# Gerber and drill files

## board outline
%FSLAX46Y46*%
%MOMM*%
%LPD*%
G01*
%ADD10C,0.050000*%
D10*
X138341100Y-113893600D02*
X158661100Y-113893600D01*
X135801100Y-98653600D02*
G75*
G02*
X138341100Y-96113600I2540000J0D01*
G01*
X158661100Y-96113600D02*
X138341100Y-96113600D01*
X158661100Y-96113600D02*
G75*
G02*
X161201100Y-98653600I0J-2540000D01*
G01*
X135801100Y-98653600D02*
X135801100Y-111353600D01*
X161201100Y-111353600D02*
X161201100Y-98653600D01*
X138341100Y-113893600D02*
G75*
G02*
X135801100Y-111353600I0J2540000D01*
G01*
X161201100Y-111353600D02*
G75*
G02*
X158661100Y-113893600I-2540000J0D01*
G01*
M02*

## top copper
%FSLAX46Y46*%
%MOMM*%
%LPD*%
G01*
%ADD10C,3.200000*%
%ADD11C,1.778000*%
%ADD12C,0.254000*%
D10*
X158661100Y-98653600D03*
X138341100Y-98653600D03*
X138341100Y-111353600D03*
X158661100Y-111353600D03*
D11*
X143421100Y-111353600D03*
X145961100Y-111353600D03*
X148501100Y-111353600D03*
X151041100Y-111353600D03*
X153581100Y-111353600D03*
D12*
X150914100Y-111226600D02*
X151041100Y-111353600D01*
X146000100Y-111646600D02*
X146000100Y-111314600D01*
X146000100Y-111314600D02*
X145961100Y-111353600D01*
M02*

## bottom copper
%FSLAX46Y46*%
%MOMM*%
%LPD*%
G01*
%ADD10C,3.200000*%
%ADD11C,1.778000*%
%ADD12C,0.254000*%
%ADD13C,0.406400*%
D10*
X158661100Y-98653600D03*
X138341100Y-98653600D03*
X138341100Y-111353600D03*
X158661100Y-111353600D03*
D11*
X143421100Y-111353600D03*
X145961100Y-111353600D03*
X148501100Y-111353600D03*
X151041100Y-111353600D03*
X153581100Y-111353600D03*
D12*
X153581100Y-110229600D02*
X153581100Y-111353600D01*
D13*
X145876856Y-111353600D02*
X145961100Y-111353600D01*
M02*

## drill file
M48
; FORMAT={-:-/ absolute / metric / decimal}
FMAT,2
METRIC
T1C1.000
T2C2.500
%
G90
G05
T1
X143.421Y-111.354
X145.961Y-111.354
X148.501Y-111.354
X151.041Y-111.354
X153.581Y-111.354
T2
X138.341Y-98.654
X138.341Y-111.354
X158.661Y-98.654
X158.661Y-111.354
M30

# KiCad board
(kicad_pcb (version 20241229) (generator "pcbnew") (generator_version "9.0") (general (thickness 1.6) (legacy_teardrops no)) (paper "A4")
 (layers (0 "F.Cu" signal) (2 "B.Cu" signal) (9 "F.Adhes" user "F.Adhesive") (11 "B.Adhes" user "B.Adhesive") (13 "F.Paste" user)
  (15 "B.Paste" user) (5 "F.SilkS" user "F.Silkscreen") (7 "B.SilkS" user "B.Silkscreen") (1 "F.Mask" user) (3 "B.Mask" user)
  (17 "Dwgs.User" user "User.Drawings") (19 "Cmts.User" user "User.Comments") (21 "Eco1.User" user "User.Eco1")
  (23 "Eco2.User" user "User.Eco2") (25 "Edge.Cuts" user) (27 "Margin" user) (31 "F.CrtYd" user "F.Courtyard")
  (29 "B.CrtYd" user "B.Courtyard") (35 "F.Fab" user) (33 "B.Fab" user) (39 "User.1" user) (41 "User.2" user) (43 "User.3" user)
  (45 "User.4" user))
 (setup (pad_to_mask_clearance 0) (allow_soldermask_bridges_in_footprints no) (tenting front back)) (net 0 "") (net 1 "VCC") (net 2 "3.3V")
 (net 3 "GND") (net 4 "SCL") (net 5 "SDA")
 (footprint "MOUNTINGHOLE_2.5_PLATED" (layer "F.Cu") (at 158.6611 98.6536)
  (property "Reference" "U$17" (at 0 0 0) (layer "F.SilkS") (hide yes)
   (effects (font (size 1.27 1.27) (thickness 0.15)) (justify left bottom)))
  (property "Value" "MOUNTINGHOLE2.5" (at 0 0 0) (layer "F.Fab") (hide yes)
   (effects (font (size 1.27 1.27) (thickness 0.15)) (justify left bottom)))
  (pad "P$1" thru_hole circle (at 0 0) (size 3.2 3.2) (drill 2.5) (layers "*.Cu" "*.Mask") (remove_unused_layers no)
   (solder_mask_margin 0.0508) (thermal_bridge_angle 0))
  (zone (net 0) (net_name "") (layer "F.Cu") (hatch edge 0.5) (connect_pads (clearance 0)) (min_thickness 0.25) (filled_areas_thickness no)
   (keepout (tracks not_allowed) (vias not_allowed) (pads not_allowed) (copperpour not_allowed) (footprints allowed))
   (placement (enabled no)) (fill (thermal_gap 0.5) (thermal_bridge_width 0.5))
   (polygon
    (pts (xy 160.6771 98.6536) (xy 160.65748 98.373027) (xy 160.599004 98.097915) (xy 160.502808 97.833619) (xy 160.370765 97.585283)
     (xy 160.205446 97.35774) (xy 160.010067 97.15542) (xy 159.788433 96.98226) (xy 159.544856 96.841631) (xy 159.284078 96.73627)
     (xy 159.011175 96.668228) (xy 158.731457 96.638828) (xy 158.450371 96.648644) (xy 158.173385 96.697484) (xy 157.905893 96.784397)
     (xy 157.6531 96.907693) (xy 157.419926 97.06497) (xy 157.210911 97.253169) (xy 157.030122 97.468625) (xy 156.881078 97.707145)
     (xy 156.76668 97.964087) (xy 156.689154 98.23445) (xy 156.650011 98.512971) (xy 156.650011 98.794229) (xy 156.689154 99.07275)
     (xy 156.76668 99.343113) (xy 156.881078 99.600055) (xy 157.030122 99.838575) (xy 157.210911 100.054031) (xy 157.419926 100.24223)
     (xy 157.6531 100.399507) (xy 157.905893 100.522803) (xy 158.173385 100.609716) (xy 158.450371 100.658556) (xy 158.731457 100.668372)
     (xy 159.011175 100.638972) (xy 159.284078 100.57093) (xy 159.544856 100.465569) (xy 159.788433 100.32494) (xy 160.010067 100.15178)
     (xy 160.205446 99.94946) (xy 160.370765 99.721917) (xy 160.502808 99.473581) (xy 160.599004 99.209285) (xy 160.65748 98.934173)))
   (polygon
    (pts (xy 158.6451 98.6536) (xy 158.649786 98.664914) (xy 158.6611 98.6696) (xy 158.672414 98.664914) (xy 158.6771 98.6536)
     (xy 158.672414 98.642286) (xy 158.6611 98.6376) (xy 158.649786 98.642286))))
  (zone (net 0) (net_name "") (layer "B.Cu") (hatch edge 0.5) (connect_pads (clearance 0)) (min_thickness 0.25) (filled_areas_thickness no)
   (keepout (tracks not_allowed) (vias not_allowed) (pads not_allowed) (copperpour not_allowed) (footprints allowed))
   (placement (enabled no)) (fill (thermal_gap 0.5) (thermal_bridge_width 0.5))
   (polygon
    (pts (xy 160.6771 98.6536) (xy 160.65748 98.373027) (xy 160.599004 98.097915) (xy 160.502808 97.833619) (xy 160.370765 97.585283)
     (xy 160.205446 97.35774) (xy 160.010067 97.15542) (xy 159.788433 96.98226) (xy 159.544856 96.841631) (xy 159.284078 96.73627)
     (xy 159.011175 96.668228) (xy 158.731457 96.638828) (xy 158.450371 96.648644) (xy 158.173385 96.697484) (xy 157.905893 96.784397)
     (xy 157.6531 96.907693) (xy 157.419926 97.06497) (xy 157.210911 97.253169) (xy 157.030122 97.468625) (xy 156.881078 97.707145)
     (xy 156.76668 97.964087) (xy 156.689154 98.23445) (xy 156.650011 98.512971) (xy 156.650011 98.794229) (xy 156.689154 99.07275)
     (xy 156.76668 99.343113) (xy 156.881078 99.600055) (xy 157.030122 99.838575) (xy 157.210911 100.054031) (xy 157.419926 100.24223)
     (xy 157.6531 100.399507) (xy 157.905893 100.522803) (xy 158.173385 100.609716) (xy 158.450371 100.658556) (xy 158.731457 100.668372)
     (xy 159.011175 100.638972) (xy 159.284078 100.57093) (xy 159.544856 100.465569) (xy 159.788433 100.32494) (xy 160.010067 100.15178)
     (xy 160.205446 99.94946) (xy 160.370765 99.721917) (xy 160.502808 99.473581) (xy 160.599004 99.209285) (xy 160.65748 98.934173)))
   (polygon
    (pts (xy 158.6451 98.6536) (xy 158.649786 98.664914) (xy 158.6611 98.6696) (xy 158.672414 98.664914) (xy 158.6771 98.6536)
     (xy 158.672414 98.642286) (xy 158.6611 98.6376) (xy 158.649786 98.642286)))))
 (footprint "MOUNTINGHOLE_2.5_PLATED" (layer "F.Cu") (at 138.3411 98.6536)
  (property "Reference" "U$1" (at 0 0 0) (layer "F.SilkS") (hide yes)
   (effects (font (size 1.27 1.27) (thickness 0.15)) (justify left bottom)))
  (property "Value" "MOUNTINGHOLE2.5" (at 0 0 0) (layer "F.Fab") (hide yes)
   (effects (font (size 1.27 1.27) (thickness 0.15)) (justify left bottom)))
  (pad "P$1" thru_hole circle (at 0 0) (size 3.2 3.2) (drill 2.5) (layers "*.Cu" "*.Mask") (remove_unused_layers no)
   (solder_mask_margin 0.0508) (thermal_bridge_angle 0))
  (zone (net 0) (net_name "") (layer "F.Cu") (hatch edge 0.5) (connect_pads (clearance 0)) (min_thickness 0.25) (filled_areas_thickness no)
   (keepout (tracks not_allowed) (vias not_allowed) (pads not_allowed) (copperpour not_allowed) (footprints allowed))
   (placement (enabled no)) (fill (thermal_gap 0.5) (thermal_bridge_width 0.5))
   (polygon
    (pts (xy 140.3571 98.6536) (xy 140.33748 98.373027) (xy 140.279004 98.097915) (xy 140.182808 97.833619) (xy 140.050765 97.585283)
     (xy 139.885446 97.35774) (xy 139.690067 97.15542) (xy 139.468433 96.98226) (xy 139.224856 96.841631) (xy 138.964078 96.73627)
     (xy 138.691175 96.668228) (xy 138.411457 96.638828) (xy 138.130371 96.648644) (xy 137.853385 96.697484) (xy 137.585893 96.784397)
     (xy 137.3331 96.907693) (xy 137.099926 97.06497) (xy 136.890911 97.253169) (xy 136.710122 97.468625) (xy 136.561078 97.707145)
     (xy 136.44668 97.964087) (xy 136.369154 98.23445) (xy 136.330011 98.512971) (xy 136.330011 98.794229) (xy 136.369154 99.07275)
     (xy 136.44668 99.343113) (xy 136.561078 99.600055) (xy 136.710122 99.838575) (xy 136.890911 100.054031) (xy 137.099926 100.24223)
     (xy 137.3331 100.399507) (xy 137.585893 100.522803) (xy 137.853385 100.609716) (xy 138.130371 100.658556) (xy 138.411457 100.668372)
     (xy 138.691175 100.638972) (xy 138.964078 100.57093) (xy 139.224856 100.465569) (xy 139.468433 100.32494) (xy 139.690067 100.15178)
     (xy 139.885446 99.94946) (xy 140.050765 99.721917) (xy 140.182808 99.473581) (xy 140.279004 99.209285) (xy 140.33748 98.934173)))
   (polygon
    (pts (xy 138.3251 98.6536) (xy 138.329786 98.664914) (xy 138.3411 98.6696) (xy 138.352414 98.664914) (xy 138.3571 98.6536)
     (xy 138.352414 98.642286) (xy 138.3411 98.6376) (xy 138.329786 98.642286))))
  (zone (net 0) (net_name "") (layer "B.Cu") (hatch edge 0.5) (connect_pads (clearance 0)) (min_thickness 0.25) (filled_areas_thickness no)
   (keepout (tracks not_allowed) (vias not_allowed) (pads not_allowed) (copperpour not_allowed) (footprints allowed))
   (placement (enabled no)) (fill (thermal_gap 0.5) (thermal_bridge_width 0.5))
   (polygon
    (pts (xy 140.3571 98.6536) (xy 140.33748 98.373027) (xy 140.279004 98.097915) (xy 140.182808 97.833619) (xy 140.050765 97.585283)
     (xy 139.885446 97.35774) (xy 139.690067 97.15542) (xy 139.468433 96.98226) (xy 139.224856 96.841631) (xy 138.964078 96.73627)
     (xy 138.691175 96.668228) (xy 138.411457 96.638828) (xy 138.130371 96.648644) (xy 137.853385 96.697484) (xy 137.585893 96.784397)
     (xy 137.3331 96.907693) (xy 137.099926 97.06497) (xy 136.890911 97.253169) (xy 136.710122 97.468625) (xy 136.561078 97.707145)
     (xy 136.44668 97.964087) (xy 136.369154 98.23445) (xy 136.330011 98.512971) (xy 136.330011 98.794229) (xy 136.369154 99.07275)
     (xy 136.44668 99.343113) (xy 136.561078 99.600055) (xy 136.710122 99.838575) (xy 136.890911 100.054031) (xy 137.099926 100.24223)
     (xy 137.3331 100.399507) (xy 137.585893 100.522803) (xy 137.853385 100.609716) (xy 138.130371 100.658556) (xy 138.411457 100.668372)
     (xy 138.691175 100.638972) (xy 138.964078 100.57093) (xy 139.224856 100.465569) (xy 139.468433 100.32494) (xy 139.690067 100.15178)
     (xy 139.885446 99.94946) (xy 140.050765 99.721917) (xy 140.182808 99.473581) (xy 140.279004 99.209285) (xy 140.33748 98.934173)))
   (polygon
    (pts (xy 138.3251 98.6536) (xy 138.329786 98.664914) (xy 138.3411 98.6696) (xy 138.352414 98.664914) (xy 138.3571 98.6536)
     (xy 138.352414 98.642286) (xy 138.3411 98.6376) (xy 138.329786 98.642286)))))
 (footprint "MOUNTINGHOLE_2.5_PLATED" (layer "F.Cu") (at 138.3411 111.3536)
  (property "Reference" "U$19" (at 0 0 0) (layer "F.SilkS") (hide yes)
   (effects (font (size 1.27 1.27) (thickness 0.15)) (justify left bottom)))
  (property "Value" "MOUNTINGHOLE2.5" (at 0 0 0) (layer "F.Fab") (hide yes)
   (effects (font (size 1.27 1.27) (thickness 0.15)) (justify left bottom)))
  (pad "P$1" thru_hole circle (at 0 0) (size 3.2 3.2) (drill 2.5) (layers "*.Cu" "*.Mask") (remove_unused_layers no)
   (solder_mask_margin 0.0508) (thermal_bridge_angle 0))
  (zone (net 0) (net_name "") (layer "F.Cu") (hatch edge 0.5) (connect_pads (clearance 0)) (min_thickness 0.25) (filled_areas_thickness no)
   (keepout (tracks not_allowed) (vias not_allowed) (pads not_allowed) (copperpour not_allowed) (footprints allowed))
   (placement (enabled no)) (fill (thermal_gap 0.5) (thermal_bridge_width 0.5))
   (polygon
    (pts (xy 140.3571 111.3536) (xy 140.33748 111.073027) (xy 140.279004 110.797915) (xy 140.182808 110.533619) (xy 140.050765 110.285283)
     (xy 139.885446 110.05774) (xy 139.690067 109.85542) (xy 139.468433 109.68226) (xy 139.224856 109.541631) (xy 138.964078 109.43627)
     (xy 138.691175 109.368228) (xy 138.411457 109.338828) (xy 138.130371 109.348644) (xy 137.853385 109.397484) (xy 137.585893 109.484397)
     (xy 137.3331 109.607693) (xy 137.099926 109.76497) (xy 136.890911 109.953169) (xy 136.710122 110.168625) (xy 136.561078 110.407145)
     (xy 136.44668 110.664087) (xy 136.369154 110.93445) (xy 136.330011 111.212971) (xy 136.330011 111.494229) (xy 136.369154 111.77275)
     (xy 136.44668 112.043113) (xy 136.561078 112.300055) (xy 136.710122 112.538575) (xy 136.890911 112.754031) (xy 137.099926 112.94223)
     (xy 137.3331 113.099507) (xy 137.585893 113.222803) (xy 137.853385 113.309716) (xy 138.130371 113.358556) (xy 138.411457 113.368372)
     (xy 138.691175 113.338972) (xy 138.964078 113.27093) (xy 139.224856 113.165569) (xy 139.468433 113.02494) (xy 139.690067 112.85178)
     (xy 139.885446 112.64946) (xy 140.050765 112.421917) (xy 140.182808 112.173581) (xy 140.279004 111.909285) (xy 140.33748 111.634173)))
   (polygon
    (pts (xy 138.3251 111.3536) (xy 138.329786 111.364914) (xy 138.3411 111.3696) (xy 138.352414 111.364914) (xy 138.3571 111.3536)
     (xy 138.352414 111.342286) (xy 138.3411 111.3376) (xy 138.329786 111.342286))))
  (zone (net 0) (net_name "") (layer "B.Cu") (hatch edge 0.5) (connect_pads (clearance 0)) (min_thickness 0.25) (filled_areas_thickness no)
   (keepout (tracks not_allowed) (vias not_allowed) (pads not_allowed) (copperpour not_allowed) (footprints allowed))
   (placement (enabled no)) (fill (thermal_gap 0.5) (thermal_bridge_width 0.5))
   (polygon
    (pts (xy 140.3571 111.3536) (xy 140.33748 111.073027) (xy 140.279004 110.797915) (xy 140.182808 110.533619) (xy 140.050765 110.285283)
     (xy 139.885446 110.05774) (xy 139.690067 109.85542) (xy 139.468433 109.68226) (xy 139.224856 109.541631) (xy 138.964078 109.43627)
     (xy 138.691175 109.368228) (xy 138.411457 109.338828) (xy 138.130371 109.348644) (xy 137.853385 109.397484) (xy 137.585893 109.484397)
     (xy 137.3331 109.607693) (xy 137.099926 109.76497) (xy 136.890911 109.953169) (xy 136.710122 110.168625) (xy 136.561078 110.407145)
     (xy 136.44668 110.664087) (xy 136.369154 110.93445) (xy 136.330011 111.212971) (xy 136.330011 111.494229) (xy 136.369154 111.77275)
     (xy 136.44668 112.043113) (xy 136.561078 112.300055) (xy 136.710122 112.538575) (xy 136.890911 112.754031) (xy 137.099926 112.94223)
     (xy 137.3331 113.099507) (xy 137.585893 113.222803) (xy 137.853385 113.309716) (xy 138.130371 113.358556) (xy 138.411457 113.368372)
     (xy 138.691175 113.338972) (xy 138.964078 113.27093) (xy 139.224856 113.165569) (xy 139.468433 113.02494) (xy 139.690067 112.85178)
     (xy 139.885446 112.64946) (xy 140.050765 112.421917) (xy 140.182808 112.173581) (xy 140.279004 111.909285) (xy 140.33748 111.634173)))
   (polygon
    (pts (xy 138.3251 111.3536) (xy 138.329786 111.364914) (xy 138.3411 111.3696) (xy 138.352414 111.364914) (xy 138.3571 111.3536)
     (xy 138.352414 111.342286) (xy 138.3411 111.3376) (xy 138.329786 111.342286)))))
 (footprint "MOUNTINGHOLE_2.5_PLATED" (layer "F.Cu") (at 158.6611 111.3536)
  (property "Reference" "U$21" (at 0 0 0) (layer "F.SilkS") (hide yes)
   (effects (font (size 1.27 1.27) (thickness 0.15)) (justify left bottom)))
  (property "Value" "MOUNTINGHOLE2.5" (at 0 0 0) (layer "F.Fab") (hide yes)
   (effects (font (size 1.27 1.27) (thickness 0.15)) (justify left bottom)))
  (pad "P$1" thru_hole circle (at 0 0) (size 3.2 3.2) (drill 2.5) (layers "*.Cu" "*.Mask") (remove_unused_layers no)
   (solder_mask_margin 0.0508) (thermal_bridge_angle 0))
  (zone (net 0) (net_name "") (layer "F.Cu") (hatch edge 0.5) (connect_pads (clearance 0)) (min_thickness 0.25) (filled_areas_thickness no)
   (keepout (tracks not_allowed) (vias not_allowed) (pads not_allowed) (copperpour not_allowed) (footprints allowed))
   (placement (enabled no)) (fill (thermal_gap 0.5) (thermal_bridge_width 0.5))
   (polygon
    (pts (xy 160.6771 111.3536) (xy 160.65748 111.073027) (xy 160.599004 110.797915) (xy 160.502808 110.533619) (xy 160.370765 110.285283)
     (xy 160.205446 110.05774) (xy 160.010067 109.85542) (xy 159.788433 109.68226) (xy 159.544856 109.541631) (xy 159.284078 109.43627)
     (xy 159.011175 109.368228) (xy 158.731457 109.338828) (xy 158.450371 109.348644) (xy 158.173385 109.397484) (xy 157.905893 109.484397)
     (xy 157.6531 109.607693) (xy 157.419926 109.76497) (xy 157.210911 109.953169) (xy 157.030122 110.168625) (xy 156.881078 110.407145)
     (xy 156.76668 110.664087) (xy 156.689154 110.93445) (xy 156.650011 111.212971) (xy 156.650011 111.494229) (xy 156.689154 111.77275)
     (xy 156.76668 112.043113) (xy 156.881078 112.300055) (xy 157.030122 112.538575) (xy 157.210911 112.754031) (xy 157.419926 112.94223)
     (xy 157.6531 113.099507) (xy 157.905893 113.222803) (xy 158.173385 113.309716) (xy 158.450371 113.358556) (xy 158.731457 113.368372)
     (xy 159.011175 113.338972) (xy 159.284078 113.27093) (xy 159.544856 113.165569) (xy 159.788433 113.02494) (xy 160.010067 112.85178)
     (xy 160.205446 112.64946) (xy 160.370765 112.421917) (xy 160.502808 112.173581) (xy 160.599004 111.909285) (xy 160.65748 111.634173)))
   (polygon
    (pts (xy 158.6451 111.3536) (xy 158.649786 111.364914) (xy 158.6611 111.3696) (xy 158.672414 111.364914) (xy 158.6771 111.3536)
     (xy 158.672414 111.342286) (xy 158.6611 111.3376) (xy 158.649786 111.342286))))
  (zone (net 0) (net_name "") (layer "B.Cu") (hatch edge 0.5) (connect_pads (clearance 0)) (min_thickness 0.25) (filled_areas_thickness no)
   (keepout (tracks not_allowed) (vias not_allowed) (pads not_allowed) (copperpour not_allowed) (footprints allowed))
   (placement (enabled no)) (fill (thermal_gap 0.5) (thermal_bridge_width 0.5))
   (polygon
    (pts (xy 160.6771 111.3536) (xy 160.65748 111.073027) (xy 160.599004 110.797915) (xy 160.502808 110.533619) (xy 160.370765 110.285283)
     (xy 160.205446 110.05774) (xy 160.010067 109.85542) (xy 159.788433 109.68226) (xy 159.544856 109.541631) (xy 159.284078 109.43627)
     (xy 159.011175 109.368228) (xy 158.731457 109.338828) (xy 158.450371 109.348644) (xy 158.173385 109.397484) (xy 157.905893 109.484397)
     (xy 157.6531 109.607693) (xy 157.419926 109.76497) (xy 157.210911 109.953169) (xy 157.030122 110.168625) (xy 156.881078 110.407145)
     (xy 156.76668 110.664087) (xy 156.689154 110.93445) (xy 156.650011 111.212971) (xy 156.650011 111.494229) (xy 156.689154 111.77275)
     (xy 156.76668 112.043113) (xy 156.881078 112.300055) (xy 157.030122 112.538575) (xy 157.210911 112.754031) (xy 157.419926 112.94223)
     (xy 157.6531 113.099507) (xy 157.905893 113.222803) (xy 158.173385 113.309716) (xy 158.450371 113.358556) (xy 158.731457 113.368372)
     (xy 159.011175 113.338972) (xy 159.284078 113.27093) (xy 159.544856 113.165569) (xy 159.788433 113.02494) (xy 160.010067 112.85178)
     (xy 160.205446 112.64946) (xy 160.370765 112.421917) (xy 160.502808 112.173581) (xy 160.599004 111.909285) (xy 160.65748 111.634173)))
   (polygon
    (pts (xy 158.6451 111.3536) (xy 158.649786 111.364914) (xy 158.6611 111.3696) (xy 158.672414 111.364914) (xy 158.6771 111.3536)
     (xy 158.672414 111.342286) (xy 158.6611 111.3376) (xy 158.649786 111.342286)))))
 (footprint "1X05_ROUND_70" (layer "F.Cu") (at 148.5011 111.3536)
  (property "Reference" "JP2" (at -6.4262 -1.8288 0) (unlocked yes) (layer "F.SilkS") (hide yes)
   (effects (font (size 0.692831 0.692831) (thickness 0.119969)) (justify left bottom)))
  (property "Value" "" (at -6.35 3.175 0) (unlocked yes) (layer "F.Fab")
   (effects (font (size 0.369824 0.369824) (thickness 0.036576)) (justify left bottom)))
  (pad "1" thru_hole circle (at -5.08 0 90) (size 1.778 1.778) (drill 1) (layers "*.Cu" "*.Mask") (remove_unused_layers no) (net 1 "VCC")
   (solder_mask_margin 0.0508) (thermal_bridge_angle 0))
  (pad "2" thru_hole circle (at -2.54 0 90) (size 1.778 1.778) (drill 1) (layers "*.Cu" "*.Mask") (remove_unused_layers no) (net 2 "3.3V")
   (solder_mask_margin 0.0508) (thermal_bridge_angle 0))
  (pad "3" thru_hole circle (at 0 0 90) (size 1.778 1.778) (drill 1) (layers "*.Cu" "*.Mask") (remove_unused_layers no) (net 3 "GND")
   (solder_mask_margin 0.0508) (thermal_bridge_angle 0))
  (pad "4" thru_hole circle (at 2.54 0 90) (size 1.778 1.778) (drill 1) (layers "*.Cu" "*.Mask") (remove_unused_layers no) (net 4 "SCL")
   (solder_mask_margin 0.0508) (thermal_bridge_angle 0))
  (pad "5" thru_hole circle (at 5.08 0 90) (size 1.778 1.778) (drill 1) (layers "*.Cu" "*.Mask") (remove_unused_layers no) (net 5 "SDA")
   (solder_mask_margin 0.0508) (thermal_bridge_angle 0)))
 (gr_line (start 138.3411 113.8936) (end 158.6611 113.8936) (stroke (width 0.05) (type solid)) (layer "Edge.Cuts"))
 (gr_arc (start 135.8011 98.6536) (mid 136.545049 96.857549) (end 138.3411 96.1136) (stroke (width 0.05) (type solid)) (layer "Edge.Cuts"))
 (gr_line (start 158.6611 96.1136) (end 138.3411 96.1136) (stroke (width 0.05) (type solid)) (layer "Edge.Cuts"))
 (gr_arc (start 158.6611 96.1136) (mid 160.457151 96.857549) (end 161.2011 98.6536) (stroke (width 0.05) (type solid)) (layer "Edge.Cuts"))
 (gr_line (start 135.8011 98.6536) (end 135.8011 111.3536) (stroke (width 0.05) (type solid)) (layer "Edge.Cuts"))
 (gr_line (start 161.2011 111.3536) (end 161.2011 98.6536) (stroke (width 0.05) (type solid)) (layer "Edge.Cuts"))
 (gr_arc (start 138.3411 113.8936) (mid 136.545049 113.149651) (end 135.8011 111.3536) (stroke (width 0.05) (type solid))
  (layer "Edge.Cuts"))
 (gr_arc (start 161.2011 111.3536) (mid 160.457151 113.149651) (end 158.6611 113.8936) (stroke (width 0.05) (type solid))
  (layer "Edge.Cuts"))
 (segment (start 153.5811 110.2296) (end 153.5811 111.3536) (width 0.254) (layer "B.Cu") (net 5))
 (segment (start 150.9141 111.2266) (end 151.0411 111.3536) (width 0.254) (layer "F.Cu") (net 4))
 (segment (start 146.0001 111.6466) (end 146.0001 111.3146) (width 0.254) (layer "F.Cu") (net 2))
 (segment (start 146.0001 111.3146) (end 145.9611 111.3536) (width 0.254) (layer "F.Cu") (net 2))
 (segment (start 145.876856 111.3536) (end 145.9611 111.3536) (width 0.4064) (layer "B.Cu") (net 2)))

